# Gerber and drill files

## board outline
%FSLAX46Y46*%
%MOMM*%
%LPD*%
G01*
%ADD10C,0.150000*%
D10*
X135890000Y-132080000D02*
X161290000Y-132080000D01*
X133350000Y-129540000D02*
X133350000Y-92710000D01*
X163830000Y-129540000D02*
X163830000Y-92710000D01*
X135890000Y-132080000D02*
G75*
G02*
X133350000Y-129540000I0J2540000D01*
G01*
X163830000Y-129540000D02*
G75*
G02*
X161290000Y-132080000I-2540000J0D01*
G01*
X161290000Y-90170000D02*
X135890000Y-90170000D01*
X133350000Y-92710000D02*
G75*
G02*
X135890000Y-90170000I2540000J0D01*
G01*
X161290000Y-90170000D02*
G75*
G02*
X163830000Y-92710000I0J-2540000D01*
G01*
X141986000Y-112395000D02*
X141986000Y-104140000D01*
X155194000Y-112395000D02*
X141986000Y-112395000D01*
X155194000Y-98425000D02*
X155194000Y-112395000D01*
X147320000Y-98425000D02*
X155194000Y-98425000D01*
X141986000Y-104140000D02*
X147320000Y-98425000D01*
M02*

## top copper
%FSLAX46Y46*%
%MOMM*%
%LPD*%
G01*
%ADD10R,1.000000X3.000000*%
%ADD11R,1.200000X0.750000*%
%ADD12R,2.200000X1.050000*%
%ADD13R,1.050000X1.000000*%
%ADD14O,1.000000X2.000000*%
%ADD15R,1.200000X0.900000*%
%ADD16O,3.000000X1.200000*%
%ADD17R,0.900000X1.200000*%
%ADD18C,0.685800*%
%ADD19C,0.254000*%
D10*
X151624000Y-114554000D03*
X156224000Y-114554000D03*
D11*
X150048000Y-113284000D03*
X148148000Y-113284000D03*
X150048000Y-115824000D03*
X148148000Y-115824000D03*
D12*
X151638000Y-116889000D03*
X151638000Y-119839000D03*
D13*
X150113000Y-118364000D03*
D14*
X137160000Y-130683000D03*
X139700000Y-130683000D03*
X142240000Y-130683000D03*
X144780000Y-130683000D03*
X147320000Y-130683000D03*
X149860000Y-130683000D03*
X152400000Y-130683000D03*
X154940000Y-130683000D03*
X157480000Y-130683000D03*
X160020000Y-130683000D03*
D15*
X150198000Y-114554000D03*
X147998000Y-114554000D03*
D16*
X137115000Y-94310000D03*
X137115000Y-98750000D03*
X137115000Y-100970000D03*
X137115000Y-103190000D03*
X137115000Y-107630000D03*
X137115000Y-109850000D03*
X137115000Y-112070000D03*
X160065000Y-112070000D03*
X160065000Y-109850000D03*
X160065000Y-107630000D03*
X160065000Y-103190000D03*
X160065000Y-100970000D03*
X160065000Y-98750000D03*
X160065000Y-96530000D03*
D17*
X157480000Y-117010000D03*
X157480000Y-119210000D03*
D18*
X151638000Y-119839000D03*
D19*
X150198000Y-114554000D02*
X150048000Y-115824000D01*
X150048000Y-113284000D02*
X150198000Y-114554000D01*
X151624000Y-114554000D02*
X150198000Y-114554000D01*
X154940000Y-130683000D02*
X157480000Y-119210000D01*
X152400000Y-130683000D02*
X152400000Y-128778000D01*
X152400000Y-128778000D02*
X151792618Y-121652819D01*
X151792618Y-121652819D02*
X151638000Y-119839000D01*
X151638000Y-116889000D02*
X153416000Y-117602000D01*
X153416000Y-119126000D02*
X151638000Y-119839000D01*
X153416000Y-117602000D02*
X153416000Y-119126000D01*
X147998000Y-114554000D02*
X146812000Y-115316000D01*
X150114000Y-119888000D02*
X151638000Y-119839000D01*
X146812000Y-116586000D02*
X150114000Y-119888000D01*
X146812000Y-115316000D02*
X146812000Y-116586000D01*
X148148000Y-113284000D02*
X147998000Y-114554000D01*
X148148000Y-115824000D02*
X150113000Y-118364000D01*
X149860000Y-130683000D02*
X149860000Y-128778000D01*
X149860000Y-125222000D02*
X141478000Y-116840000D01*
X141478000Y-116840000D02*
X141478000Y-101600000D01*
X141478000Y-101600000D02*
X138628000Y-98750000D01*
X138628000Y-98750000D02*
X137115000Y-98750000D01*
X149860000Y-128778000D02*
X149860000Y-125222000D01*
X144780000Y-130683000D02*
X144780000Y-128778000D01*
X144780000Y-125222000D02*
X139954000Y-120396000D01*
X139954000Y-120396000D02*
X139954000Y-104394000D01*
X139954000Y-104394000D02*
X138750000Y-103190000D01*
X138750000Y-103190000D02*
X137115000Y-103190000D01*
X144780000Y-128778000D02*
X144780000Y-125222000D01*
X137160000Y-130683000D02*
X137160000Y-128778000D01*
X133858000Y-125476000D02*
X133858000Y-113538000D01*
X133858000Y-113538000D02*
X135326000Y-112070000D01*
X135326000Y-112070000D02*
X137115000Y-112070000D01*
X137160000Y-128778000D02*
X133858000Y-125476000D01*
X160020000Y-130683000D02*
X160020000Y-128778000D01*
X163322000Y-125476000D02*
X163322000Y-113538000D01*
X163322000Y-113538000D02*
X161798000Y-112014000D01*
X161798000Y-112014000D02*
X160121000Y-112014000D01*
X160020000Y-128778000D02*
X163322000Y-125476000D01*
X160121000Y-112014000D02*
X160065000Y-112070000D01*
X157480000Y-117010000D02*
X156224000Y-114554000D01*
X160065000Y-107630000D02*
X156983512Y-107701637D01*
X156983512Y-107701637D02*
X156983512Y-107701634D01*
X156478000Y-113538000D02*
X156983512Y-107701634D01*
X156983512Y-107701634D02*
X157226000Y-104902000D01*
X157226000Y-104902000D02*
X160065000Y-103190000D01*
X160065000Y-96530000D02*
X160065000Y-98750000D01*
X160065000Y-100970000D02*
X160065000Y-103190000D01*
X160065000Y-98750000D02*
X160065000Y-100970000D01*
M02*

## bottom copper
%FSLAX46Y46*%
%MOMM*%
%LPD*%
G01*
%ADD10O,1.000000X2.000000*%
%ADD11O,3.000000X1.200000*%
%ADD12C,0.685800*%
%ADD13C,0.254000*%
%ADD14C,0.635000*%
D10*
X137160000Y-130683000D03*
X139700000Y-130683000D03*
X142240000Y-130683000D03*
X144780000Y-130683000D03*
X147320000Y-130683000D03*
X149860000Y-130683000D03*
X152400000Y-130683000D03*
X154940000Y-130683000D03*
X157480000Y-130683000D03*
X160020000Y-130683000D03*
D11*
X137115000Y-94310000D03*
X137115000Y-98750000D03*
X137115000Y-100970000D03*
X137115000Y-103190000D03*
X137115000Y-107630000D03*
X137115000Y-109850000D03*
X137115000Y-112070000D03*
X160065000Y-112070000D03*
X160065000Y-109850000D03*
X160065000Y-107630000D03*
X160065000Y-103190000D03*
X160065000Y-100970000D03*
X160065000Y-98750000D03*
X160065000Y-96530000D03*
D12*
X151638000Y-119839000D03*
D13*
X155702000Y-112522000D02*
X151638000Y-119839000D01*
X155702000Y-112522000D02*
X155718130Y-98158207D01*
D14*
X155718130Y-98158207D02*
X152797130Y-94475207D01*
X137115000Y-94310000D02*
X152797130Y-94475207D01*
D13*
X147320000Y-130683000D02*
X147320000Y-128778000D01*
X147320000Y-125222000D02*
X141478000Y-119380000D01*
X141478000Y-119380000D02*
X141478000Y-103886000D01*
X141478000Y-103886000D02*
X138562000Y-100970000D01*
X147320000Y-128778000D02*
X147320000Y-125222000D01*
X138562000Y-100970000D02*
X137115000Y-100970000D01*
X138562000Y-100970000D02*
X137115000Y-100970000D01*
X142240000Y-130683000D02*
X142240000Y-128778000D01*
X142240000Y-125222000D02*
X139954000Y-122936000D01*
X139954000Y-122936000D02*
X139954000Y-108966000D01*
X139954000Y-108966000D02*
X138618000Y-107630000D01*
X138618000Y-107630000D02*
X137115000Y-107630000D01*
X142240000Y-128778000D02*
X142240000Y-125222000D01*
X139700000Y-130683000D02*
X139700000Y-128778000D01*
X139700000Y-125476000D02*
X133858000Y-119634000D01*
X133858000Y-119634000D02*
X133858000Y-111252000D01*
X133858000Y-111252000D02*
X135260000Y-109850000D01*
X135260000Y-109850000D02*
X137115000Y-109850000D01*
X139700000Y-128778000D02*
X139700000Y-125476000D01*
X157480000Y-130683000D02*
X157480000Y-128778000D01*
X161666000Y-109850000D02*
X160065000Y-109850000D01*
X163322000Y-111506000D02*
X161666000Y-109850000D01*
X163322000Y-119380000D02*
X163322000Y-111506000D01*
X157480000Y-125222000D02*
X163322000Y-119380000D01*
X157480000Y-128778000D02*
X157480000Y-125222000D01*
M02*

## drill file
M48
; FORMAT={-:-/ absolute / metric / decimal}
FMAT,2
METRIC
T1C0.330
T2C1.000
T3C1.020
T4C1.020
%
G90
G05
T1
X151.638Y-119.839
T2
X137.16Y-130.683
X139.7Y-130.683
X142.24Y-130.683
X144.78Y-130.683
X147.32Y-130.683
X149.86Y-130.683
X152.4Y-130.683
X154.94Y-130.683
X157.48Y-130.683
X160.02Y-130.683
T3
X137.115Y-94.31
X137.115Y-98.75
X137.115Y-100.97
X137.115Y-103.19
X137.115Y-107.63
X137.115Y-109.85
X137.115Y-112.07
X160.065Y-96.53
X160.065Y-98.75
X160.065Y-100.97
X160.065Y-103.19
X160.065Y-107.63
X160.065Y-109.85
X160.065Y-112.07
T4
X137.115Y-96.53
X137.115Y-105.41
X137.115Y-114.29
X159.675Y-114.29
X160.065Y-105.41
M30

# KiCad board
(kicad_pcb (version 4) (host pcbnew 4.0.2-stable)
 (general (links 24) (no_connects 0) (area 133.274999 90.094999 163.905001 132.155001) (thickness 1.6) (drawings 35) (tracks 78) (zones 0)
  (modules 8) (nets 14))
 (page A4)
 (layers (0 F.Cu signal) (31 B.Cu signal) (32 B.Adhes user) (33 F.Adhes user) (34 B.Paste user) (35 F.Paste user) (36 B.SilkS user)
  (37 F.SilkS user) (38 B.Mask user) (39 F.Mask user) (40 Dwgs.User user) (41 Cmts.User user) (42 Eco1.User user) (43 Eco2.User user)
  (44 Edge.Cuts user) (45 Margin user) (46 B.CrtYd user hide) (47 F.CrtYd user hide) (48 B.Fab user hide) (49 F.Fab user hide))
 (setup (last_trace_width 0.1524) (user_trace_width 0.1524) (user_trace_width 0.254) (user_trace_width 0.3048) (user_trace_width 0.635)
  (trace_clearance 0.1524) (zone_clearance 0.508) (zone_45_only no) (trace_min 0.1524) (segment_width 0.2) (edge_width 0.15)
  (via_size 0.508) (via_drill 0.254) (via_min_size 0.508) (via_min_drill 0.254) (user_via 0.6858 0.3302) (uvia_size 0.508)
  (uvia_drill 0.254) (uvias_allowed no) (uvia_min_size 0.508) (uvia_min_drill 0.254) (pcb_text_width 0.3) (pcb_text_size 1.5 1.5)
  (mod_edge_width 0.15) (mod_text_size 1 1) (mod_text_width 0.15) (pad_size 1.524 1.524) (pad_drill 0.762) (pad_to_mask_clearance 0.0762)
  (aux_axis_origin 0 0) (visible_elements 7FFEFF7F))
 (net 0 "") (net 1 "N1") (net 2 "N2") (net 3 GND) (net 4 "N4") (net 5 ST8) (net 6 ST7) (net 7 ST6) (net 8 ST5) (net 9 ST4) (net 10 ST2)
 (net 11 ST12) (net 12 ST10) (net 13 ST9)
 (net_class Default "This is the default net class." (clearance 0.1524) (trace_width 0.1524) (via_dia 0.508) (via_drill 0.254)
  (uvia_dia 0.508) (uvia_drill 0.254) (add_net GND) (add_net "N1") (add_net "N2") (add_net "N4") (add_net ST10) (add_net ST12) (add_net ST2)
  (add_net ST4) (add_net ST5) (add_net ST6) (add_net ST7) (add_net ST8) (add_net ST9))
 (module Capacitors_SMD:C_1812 (layer F.Cu) (at 153.924 114.554)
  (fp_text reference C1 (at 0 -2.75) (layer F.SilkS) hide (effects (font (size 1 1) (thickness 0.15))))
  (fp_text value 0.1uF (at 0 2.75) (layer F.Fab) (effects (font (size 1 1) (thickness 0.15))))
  (pad 1 smd rect (at -2.3 0) (size 1 3) (layers F.Cu F.Paste F.Mask) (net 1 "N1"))
  (pad 2 smd rect (at 2.3 0) (size 1 3) (layers F.Cu F.Paste F.Mask) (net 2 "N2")))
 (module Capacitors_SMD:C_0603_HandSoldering (layer F.Cu) (at 149.098 113.284 180)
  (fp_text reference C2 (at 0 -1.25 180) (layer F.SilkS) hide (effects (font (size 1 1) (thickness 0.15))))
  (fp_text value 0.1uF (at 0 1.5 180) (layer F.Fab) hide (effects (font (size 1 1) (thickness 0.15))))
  (pad 1 smd rect (at -0.95 0 180) (size 1.2 0.75) (layers F.Cu F.Paste F.Mask) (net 1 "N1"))
  (pad 2 smd rect (at 0.95 0 180) (size 1.2 0.75) (layers F.Cu F.Paste F.Mask) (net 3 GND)))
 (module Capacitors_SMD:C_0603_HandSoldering (layer F.Cu) (at 149.098 115.824 180)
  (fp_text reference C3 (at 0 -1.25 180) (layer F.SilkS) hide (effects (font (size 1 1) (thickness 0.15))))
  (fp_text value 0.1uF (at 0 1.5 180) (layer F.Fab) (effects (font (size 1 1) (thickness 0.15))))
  (pad 1 smd rect (at -0.95 0 180) (size 1.2 0.75) (layers F.Cu F.Paste F.Mask) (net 1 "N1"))
  (pad 2 smd rect (at 0.95 0 180) (size 1.2 0.75) (layers F.Cu F.Paste F.Mask) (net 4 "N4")))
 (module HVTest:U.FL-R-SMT (layer F.Cu) (at 151.638 118.364 270)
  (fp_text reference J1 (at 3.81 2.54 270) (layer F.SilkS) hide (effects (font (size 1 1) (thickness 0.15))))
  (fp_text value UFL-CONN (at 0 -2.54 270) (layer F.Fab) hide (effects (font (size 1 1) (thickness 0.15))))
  (pad 2 smd rect (at -1.475 0 270) (size 1.05 2.2) (layers F.Cu F.Paste F.Mask) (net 3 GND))
  (pad 3 smd rect (at 1.475 0 270) (size 1.05 2.2) (layers F.Cu F.Paste F.Mask) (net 3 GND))
  (pad 1 smd rect (at 0 1.525 270) (size 1 1.05) (layers F.Cu F.Paste F.Mask) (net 4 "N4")))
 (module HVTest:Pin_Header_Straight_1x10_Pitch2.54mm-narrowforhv (layer F.Cu) (at 137.16 130.683 90)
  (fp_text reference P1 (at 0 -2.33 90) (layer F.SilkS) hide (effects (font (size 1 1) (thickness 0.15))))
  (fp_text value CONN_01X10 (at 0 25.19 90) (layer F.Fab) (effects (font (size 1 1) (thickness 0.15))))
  (pad 1 thru_hole oval (at 0 0 90) (size 2 1) (drill 1) (layers *.Cu *.Mask) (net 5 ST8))
  (pad 2 thru_hole oval (at 0 2.54 90) (size 2 1) (drill 1) (layers *.Cu *.Mask) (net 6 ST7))
  (pad 3 thru_hole oval (at 0 5.08 90) (size 2 1) (drill 1) (layers *.Cu *.Mask) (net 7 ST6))
  (pad 4 thru_hole oval (at 0 7.62 90) (size 2 1) (drill 1) (layers *.Cu *.Mask) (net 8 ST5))
  (pad 5 thru_hole oval (at 0 10.16 90) (size 2 1) (drill 1) (layers *.Cu *.Mask) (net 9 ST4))
  (pad 6 thru_hole oval (at 0 12.7 90) (size 2 1) (drill 1) (layers *.Cu *.Mask) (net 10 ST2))
  (pad 7 thru_hole oval (at 0 15.24 90) (size 2 1) (drill 1) (layers *.Cu *.Mask) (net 3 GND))
  (pad 8 thru_hole oval (at 0 17.78 90) (size 2 1) (drill 1) (layers *.Cu *.Mask) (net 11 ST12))
  (pad 9 thru_hole oval (at 0 20.32 90) (size 2 1) (drill 1) (layers *.Cu *.Mask) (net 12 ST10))
  (pad 10 thru_hole oval (at 0 22.86 90) (size 2 1) (drill 1) (layers *.Cu *.Mask) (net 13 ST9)))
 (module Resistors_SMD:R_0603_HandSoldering (layer F.Cu) (at 149.098 114.554 180)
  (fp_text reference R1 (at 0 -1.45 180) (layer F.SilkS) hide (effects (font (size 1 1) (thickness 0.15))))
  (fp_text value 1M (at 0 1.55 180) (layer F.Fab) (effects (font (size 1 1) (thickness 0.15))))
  (pad 1 smd rect (at -1.1 0 180) (size 1.2 0.9) (layers F.Cu F.Paste F.Mask) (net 1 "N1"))
  (pad 2 smd rect (at 1.1 0 180) (size 1.2 0.9) (layers F.Cu F.Paste F.Mask) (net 3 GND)))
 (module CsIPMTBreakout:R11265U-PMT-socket (layer F.Cu) (at 148.59 105.41)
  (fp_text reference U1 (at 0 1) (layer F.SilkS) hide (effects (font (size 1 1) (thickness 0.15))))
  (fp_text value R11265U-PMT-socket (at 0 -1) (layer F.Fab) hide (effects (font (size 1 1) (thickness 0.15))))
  (pad 1 thru_hole oval (at -11.475 -11.1) (size 3 1.2) (drill 1.02) (layers *.Cu *.Mask F.SilkS) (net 3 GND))
  (pad "" np_thru_hole oval (at -11.475 -8.88) (size 1.02 1.02) (drill 1.02) (layers *.Cu *.Mask F.SilkS))
  (pad 2 thru_hole oval (at -11.475 -6.66) (size 3 1.2) (drill 1.02) (layers *.Cu *.Mask F.SilkS) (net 10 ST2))
  (pad 3 thru_hole oval (at -11.475 -4.44) (size 3 1.2) (drill 1.02) (layers *.Cu *.Mask F.SilkS) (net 9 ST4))
  (pad 4 thru_hole oval (at -11.475 -2.22) (size 3 1.2) (drill 1.02) (layers *.Cu *.Mask F.SilkS) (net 8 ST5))
  (pad "" np_thru_hole oval (at -11.475 0) (size 1.02 1.02) (drill 1.02) (layers *.Cu *.Mask F.SilkS))
  (pad 5 thru_hole oval (at -11.475 2.22) (size 3 1.2) (drill 1.02) (layers *.Cu *.Mask F.SilkS) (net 7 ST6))
  (pad 6 thru_hole oval (at -11.475 4.44) (size 3 1.2) (drill 1.02) (layers *.Cu *.Mask F.SilkS) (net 6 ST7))
  (pad 7 thru_hole oval (at -11.475 6.66) (size 3 1.2) (drill 1.02) (layers *.Cu *.Mask F.SilkS) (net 5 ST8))
  (pad "" np_thru_hole oval (at -11.475 8.88) (size 1.02 1.02) (drill 1.02) (layers *.Cu *.Mask F.SilkS))
  (pad "" np_thru_hole oval (at 11.085 8.88) (size 1.02 1.02) (drill 1.02) (layers *.Cu *.Mask F.SilkS))
  (pad 8 thru_hole oval (at 11.475 6.66) (size 3 1.2) (drill 1.02) (layers *.Cu *.Mask F.SilkS) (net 13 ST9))
  (pad 9 thru_hole oval (at 11.475 4.44) (size 3 1.2) (drill 1.02) (layers *.Cu *.Mask F.SilkS) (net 12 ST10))
  (pad 10 thru_hole oval (at 11.475 2.22) (size 3 1.2) (drill 1.02) (layers *.Cu *.Mask F.SilkS) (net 2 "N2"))
  (pad "" np_thru_hole oval (at 11.475 0) (size 1.02 1.02) (drill 1.02) (layers *.Cu *.Mask F.SilkS))
  (pad 11 thru_hole oval (at 11.475 -2.22) (size 3 1.2) (drill 1.02) (layers *.Cu *.Mask F.SilkS) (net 2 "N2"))
  (pad 12 thru_hole oval (at 11.475 -4.44) (size 3 1.2) (drill 1.02) (layers *.Cu *.Mask F.SilkS) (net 2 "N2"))
  (pad 13 thru_hole oval (at 11.475 -6.66) (size 3 1.2) (drill 1.02) (layers *.Cu *.Mask F.SilkS) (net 2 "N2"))
  (pad 14 thru_hole oval (at 11.475 -8.88) (size 3 1.2) (drill 1.02) (layers *.Cu *.Mask F.SilkS) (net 2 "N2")))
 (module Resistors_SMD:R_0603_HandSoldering (layer F.Cu) (at 157.48 118.11 270)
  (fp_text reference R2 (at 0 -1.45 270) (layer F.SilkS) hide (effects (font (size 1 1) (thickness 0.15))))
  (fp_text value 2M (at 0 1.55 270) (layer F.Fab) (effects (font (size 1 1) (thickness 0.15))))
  (pad 1 smd rect (at -1.1 0 270) (size 1.2 0.9) (layers F.Cu F.Paste F.Mask) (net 2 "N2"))
  (pad 2 smd rect (at 1.1 0 270) (size 1.2 0.9) (layers F.Cu F.Paste F.Mask) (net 11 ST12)))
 (gr_line (start 135.89 132.08) (end 161.29 132.08) (angle 90) (layer Edge.Cuts) (width 0.15))
 (gr_line (start 133.35 129.54) (end 133.35 92.71) (angle 90) (layer Edge.Cuts) (width 0.15))
 (gr_line (start 163.83 129.54) (end 163.83 92.71) (angle 90) (layer Edge.Cuts) (width 0.15))
 (gr_arc (start 135.89 129.54) (end 135.89 132.08) (angle 90) (layer Edge.Cuts) (width 0.15))
 (gr_arc (start 161.29 129.54) (end 163.83 129.54) (angle 90) (layer Edge.Cuts) (width 0.15))
 (gr_line (start 161.29 90.17) (end 135.89 90.17) (angle 90) (layer Edge.Cuts) (width 0.15))
 (gr_arc (start 135.89 92.71) (end 133.35 92.71) (angle 90) (layer Edge.Cuts) (width 0.15))
 (gr_arc (start 161.29 92.71) (end 161.29 90.17) (angle 90) (layer Edge.Cuts) (width 0.15))
 (gr_line (start 141.986 112.395) (end 141.986 104.14) (angle 90) (layer Edge.Cuts) (width 0.15))
 (gr_line (start 155.194 112.395) (end 141.986 112.395) (angle 90) (layer Edge.Cuts) (width 0.15))
 (gr_line (start 155.194 98.425) (end 155.194 112.395) (angle 90) (layer Edge.Cuts) (width 0.15))
 (gr_line (start 147.32 98.425) (end 155.194 98.425) (angle 90) (layer Edge.Cuts) (width 0.15))
 (gr_line (start 141.986 104.14) (end 147.32 98.425) (angle 90) (layer Edge.Cuts) (width 0.15))
 (segment (start 150.198 114.554) (end 150.048 115.824) (width 0.254) (layer F.Cu) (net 1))
 (segment (start 150.048 113.284) (end 150.198 114.554) (width 0.254) (layer F.Cu) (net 1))
 (segment (start 151.624 114.554) (end 150.198 114.554) (width 0.254) (layer F.Cu) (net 1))
 (segment (start 154.94 130.683) (end 157.48 119.21) (width 0.254) (layer F.Cu) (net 11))
 (segment (start 152.4 130.683) (end 152.4 128.778) (width 0.254) (layer F.Cu) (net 3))
 (segment (start 152.4 128.778) (end 151.792618 121.652819) (width 0.254) (layer F.Cu) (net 3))
 (segment (start 151.792618 121.652819) (end 151.638 119.839) (width 0.254) (layer F.Cu) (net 3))
 (segment (start 151.638 116.889) (end 153.416 117.602) (width 0.254) (layer F.Cu) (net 3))
 (segment (start 153.416 119.126) (end 151.638 119.839) (width 0.254) (layer F.Cu) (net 3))
 (segment (start 153.416 117.602) (end 153.416 119.126) (width 0.254) (layer F.Cu) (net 3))
 (segment (start 147.998 114.554) (end 146.812 115.316) (width 0.254) (layer F.Cu) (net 3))
 (segment (start 150.114 119.888) (end 151.638 119.839) (width 0.254) (layer F.Cu) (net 3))
 (segment (start 146.812 116.586) (end 150.114 119.888) (width 0.254) (layer F.Cu) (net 3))
 (segment (start 146.812 115.316) (end 146.812 116.586) (width 0.254) (layer F.Cu) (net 3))
 (segment (start 148.148 113.284) (end 147.998 114.554) (width 0.254) (layer F.Cu) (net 3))
 (via (at 151.638 119.839) (size 0.6858) (drill 0.3302) (layers F.Cu B.Cu) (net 3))
 (segment (start 155.702 112.522) (end 151.638 119.839) (width 0.254) (layer B.Cu) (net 3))
 (segment (start 155.702 112.522) (end 155.71813 98.158207) (width 0.254) (layer B.Cu) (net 3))
 (segment (start 155.71813 98.158207) (end 152.79713 94.475207) (width 0.635) (layer B.Cu) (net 3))
 (segment (start 137.115 94.31) (end 152.79713 94.475207) (width 0.635) (layer B.Cu) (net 3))
 (segment (start 148.148 115.824) (end 150.113 118.364) (width 0.254) (layer F.Cu) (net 4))
 (segment (start 149.86 130.683) (end 149.86 128.778) (width 0.254) (layer F.Cu) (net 10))
 (segment (start 149.86 125.222) (end 141.478 116.84) (width 0.254) (layer F.Cu) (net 10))
 (segment (start 141.478 116.84) (end 141.478 101.6) (width 0.254) (layer F.Cu) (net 10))
 (segment (start 141.478 101.6) (end 138.628 98.75) (width 0.254) (layer F.Cu) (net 10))
 (segment (start 138.628 98.75) (end 137.115 98.75) (width 0.254) (layer F.Cu) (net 10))
 (segment (start 149.86 128.778) (end 149.86 125.222) (width 0.254) (layer F.Cu) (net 10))
 (segment (start 147.32 130.683) (end 147.32 128.778) (width 0.254) (layer B.Cu) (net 9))
 (segment (start 147.32 125.222) (end 141.478 119.38) (width 0.254) (layer B.Cu) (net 9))
 (segment (start 141.478 119.38) (end 141.478 103.886) (width 0.254) (layer B.Cu) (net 9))
 (segment (start 141.478 103.886) (end 138.562 100.97) (width 0.254) (layer B.Cu) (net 9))
 (segment (start 147.32 128.778) (end 147.32 125.222) (width 0.254) (layer B.Cu) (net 9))
 (segment (start 138.562 100.97) (end 137.115 100.97) (width 0.254) (layer B.Cu) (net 9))
 (segment (start 138.562 100.97) (end 137.115 100.97) (width 0.254) (layer B.Cu) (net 9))
 (segment (start 144.78 130.683) (end 144.78 128.778) (width 0.254) (layer F.Cu) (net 8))
 (segment (start 144.78 125.222) (end 139.954 120.396) (width 0.254) (layer F.Cu) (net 8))
 (segment (start 139.954 120.396) (end 139.954 104.394) (width 0.254) (layer F.Cu) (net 8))
 (segment (start 139.954 104.394) (end 138.75 103.19) (width 0.254) (layer F.Cu) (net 8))
 (segment (start 138.75 103.19) (end 137.115 103.19) (width 0.254) (layer F.Cu) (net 8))
 (segment (start 144.78 128.778) (end 144.78 125.222) (width 0.254) (layer F.Cu) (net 8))
 (segment (start 142.24 130.683) (end 142.24 128.778) (width 0.254) (layer B.Cu) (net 7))
 (segment (start 142.24 125.222) (end 139.954 122.936) (width 0.254) (layer B.Cu) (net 7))
 (segment (start 139.954 122.936) (end 139.954 108.966) (width 0.254) (layer B.Cu) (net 7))
 (segment (start 139.954 108.966) (end 138.618 107.63) (width 0.254) (layer B.Cu) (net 7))
 (segment (start 138.618 107.63) (end 137.115 107.63) (width 0.254) (layer B.Cu) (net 7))
 (segment (start 142.24 128.778) (end 142.24 125.222) (width 0.254) (layer B.Cu) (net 7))
 (segment (start 139.7 130.683) (end 139.7 128.778) (width 0.254) (layer B.Cu) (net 6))
 (segment (start 139.7 125.476) (end 133.858 119.634) (width 0.254) (layer B.Cu) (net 6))
 (segment (start 133.858 119.634) (end 133.858 111.252) (width 0.254) (layer B.Cu) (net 6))
 (segment (start 133.858 111.252) (end 135.26 109.85) (width 0.254) (layer B.Cu) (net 6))
 (segment (start 135.26 109.85) (end 137.115 109.85) (width 0.254) (layer B.Cu) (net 6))
 (segment (start 139.7 128.778) (end 139.7 125.476) (width 0.254) (layer B.Cu) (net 6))
 (segment (start 137.16 130.683) (end 137.16 128.778) (width 0.254) (layer F.Cu) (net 5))
 (segment (start 133.858 125.476) (end 133.858 113.538) (width 0.254) (layer F.Cu) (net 5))
 (segment (start 133.858 113.538) (end 135.326 112.07) (width 0.254) (layer F.Cu) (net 5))
 (segment (start 135.326 112.07) (end 137.115 112.07) (width 0.254) (layer F.Cu) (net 5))
 (segment (start 137.16 128.778) (end 133.858 125.476) (width 0.254) (layer F.Cu) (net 5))
 (segment (start 160.02 130.683) (end 160.02 128.778) (width 0.254) (layer F.Cu) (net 13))
 (segment (start 163.322 125.476) (end 163.322 113.538) (width 0.254) (layer F.Cu) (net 13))
 (segment (start 163.322 113.538) (end 161.798 112.014) (width 0.254) (layer F.Cu) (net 13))
 (segment (start 161.798 112.014) (end 160.121 112.014) (width 0.254) (layer F.Cu) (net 13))
 (segment (start 160.02 128.778) (end 163.322 125.476) (width 0.254) (layer F.Cu) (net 13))
 (segment (start 160.121 112.014) (end 160.065 112.07) (width 0.254) (layer F.Cu) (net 13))
 (segment (start 157.48 130.683) (end 157.48 128.778) (width 0.254) (layer B.Cu) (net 12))
 (segment (start 161.666 109.85) (end 160.065 109.85) (width 0.254) (layer B.Cu) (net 12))
 (segment (start 163.322 111.506) (end 161.666 109.85) (width 0.254) (layer B.Cu) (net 12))
 (segment (start 163.322 119.38) (end 163.322 111.506) (width 0.254) (layer B.Cu) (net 12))
 (segment (start 157.48 125.222) (end 163.322 119.38) (width 0.254) (layer B.Cu) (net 12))
 (segment (start 157.48 128.778) (end 157.48 125.222) (width 0.254) (layer B.Cu) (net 12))
 (segment (start 157.48 117.01) (end 156.224 114.554) (width 0.254) (layer F.Cu) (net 2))
 (segment (start 160.065 107.63) (end 156.983512 107.701637) (width 0.254) (layer F.Cu) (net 2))
 (segment (start 156.983512 107.701637) (end 156.983512 107.701634) (width 0.254) (layer F.Cu) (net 2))
 (segment (start 156.478 113.538) (end 156.983512 107.701634) (width 0.254) (layer F.Cu) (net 2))
 (segment (start 156.983512 107.701634) (end 157.226 104.902) (width 0.254) (layer F.Cu) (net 2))
 (segment (start 157.226 104.902) (end 160.065 103.19) (width 0.254) (layer F.Cu) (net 2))
 (segment (start 160.065 96.53) (end 160.065 98.75) (width 0.254) (layer F.Cu) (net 2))
 (segment (start 160.065 100.97) (end 160.065 103.19) (width 0.254) (layer F.Cu) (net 2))
 (segment (start 160.065 98.75) (end 160.065 100.97) (width 0.254) (layer F.Cu) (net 2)))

